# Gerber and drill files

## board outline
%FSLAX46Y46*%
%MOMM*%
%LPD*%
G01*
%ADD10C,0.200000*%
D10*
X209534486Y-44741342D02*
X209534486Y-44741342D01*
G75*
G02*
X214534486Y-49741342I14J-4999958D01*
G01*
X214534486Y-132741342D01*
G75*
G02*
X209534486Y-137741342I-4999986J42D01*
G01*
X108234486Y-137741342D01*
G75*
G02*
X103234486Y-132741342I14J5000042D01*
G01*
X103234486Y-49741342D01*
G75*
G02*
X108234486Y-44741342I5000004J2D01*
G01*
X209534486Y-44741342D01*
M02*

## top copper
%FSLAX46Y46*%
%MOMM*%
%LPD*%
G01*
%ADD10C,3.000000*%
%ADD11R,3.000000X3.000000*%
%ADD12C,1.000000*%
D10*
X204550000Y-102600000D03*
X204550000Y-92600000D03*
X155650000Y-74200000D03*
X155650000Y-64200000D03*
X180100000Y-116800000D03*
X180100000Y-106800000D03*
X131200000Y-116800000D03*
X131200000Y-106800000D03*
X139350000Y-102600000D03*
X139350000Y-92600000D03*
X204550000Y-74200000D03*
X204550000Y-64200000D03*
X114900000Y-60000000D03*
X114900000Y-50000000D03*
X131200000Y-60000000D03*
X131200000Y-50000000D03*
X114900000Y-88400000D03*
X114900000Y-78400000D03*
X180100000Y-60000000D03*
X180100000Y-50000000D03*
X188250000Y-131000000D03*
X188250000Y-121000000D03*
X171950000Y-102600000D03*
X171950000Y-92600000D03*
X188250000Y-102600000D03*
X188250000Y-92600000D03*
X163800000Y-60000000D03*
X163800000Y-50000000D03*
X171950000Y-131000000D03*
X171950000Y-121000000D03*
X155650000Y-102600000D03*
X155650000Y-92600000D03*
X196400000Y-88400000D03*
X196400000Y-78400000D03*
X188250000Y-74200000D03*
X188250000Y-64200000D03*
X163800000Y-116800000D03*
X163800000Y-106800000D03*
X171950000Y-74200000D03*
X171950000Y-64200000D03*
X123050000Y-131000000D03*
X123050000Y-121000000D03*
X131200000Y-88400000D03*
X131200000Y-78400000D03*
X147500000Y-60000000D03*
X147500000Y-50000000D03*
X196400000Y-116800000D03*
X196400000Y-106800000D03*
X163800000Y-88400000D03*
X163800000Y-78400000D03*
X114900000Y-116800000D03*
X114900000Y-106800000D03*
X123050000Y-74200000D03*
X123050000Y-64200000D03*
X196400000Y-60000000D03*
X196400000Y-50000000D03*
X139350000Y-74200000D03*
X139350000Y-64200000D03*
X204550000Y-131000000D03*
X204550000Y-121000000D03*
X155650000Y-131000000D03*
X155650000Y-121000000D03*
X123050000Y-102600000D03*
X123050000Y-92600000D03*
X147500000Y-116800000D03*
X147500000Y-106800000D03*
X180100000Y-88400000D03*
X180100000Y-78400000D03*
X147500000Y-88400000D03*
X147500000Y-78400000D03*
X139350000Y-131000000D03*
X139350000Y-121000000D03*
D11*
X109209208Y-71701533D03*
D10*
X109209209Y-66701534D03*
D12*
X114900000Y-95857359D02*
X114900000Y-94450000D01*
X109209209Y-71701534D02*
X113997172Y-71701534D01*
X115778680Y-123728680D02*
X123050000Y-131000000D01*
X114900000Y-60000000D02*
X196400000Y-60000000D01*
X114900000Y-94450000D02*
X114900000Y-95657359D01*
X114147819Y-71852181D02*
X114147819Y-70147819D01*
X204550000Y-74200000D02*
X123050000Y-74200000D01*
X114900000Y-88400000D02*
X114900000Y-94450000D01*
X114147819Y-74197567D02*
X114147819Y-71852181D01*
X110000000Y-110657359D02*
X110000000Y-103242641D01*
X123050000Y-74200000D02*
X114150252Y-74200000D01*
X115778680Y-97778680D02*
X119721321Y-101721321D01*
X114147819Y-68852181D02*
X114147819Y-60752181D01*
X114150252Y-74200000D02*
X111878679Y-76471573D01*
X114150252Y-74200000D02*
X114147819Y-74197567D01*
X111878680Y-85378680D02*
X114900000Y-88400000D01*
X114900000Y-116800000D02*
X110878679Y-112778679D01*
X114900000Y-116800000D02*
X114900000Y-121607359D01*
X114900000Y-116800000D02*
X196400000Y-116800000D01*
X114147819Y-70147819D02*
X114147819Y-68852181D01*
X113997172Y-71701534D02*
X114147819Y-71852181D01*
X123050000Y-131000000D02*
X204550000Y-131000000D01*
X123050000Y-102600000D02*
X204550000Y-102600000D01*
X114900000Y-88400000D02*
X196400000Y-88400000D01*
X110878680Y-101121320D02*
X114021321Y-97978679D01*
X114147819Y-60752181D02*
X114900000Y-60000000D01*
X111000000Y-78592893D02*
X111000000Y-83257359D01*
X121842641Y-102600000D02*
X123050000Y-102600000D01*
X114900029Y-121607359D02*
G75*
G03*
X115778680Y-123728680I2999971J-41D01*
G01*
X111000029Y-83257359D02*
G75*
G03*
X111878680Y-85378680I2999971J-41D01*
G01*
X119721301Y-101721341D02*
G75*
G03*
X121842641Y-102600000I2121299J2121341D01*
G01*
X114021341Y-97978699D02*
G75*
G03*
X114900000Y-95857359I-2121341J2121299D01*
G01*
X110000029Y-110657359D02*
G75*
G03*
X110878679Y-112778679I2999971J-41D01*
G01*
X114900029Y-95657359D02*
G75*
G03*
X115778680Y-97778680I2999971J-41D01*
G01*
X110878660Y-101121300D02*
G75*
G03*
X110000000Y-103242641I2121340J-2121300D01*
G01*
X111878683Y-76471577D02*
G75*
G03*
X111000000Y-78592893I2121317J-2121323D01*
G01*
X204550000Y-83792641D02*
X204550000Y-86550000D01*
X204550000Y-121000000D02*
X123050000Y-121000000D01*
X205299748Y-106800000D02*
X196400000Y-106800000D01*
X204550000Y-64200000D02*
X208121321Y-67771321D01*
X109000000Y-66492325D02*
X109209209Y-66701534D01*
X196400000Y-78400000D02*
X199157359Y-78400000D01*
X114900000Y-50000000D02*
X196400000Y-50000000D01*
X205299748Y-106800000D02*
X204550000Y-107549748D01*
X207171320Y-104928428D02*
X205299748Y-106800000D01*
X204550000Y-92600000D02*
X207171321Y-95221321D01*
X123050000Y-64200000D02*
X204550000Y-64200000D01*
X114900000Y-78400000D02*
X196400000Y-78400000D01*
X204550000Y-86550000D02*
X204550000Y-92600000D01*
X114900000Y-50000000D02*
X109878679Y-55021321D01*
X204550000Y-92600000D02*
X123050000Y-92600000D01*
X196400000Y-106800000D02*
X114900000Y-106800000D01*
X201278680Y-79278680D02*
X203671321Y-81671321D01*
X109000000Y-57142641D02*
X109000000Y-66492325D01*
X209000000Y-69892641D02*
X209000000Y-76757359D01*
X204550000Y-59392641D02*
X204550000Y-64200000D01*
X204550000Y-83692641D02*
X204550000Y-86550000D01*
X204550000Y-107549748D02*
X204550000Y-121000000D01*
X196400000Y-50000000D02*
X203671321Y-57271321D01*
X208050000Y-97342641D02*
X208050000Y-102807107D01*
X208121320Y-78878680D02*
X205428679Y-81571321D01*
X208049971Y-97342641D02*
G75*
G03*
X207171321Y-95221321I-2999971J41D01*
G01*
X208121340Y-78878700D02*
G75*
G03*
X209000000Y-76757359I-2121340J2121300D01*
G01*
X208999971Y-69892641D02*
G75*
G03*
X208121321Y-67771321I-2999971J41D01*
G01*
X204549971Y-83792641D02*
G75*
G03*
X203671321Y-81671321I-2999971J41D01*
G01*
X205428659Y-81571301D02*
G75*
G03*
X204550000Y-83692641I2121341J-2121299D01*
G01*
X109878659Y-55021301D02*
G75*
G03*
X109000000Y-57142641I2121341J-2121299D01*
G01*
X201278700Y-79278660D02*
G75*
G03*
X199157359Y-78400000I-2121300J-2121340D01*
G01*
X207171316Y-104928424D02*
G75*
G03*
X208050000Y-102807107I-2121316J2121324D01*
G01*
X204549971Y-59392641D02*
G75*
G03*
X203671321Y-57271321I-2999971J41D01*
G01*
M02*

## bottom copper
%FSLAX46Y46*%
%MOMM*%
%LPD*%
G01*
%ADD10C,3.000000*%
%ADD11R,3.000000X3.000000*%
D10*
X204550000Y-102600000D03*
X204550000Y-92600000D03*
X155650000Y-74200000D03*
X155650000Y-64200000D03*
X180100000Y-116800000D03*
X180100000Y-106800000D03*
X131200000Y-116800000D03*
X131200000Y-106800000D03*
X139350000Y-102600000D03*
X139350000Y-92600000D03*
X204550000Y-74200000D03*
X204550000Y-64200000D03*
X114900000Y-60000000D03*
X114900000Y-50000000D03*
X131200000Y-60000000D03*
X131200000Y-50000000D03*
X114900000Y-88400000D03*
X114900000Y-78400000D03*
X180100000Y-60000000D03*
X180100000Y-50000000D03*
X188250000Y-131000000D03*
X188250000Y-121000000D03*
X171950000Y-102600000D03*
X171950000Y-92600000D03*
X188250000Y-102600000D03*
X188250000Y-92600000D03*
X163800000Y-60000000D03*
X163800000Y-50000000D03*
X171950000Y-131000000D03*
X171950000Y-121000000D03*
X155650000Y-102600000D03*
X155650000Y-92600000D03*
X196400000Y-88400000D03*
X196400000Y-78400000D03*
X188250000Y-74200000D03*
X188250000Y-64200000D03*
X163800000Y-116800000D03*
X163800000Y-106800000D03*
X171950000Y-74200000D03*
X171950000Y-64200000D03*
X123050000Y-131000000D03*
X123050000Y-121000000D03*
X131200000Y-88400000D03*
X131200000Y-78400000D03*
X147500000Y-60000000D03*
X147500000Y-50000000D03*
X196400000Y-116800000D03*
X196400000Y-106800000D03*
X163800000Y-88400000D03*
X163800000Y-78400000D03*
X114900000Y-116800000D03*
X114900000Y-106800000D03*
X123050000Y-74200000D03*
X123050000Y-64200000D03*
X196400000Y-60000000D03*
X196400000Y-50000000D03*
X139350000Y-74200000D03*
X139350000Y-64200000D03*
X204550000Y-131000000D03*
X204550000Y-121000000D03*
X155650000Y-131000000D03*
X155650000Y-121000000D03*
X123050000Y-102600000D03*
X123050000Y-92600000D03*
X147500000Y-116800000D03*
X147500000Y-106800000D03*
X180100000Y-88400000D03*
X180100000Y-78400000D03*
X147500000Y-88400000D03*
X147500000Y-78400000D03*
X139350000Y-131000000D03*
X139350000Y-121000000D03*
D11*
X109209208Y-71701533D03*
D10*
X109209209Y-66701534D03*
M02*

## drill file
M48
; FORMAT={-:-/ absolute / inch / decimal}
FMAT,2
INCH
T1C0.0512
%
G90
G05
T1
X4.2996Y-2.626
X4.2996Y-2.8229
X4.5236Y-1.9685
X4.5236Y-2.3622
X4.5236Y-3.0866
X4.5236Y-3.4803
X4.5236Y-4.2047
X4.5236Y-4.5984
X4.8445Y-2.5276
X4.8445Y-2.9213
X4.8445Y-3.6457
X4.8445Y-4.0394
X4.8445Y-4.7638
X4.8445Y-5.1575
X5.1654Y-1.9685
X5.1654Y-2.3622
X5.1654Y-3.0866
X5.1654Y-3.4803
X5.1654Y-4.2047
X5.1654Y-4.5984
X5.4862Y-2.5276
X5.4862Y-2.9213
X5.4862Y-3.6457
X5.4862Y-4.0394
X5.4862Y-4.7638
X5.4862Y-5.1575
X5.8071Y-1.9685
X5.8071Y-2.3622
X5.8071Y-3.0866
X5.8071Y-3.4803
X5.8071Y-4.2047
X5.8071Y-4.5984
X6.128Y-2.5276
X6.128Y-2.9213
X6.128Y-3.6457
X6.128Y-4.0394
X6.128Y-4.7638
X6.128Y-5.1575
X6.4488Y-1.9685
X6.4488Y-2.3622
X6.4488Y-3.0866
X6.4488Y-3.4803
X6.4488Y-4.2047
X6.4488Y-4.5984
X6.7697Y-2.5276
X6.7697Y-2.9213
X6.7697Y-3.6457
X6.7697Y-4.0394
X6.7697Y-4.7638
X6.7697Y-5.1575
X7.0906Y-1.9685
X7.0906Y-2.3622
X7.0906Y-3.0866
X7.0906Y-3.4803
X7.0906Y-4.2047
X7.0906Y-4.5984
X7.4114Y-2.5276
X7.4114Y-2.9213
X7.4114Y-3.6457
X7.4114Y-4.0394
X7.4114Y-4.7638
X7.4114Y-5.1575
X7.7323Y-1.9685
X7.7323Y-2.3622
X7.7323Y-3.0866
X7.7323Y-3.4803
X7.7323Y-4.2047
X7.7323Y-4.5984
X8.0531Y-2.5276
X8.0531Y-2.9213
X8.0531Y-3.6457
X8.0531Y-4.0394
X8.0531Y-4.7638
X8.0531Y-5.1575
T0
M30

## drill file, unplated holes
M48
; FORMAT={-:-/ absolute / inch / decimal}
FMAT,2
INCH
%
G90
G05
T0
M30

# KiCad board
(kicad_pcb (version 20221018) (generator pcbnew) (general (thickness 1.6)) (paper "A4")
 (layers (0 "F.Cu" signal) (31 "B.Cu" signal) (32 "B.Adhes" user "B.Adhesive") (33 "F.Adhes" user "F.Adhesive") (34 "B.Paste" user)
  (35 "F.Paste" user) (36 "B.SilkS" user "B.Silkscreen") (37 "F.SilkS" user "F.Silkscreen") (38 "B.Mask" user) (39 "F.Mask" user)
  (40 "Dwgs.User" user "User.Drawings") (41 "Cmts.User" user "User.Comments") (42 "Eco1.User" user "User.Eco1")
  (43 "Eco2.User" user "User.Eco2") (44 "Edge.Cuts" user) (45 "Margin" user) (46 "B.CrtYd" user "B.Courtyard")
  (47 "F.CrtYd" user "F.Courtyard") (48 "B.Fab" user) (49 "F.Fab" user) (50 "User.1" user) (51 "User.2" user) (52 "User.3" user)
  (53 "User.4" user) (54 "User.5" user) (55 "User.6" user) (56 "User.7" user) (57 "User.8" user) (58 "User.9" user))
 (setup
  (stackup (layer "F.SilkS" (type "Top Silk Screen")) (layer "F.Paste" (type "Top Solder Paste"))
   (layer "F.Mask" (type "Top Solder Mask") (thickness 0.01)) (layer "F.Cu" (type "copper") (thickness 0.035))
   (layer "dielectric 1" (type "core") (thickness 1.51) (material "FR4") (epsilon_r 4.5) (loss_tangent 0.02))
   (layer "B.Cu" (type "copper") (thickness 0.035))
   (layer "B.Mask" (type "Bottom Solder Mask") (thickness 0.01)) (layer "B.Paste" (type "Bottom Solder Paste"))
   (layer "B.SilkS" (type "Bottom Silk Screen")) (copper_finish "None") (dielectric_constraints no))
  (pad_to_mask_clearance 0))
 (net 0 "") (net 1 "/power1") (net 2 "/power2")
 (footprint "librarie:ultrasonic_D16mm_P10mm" (layer "F.Cu") (at 204.55 97.6)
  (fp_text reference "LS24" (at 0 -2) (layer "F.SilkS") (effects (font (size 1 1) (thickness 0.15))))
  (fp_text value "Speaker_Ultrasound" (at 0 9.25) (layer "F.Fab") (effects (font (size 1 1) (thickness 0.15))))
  (pad "1" thru_hole circle (at 0 5) (size 3 3) (drill 1.3) (layers "*.Cu" "*.Mask") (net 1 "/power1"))
  (pad "2" thru_hole circle (at 0 -5) (size 3 3) (drill 1.3) (layers "*.Cu" "*.Mask") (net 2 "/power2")))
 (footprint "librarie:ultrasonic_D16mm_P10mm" (layer "F.Cu") (at 155.65 69.2)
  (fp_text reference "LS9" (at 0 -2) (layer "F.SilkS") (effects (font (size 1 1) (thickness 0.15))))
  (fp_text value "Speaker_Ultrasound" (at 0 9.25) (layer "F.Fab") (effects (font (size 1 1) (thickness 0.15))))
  (pad "1" thru_hole circle (at 0 5) (size 3 3) (drill 1.3) (layers "*.Cu" "*.Mask") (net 1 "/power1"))
  (pad "2" thru_hole circle (at 0 -5) (size 3 3) (drill 1.3) (layers "*.Cu" "*.Mask") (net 2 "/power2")))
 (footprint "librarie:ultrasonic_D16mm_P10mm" (layer "F.Cu") (at 180.1 111.8)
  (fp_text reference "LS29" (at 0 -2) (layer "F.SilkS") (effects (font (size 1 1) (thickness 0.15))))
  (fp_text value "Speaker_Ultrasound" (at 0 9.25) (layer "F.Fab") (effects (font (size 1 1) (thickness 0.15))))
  (pad "1" thru_hole circle (at 0 5) (size 3 3) (drill 1.3) (layers "*.Cu" "*.Mask") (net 1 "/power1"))
  (pad "2" thru_hole circle (at 0 -5) (size 3 3) (drill 1.3) (layers "*.Cu" "*.Mask") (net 2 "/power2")))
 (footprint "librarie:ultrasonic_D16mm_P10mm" (layer "F.Cu") (at 131.2 111.8)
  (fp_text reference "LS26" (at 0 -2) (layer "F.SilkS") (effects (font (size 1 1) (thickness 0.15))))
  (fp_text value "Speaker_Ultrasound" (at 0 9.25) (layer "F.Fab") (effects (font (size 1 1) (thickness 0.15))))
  (pad "1" thru_hole circle (at 0 5) (size 3 3) (drill 1.3) (layers "*.Cu" "*.Mask") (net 1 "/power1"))
  (pad "2" thru_hole circle (at 0 -5) (size 3 3) (drill 1.3) (layers "*.Cu" "*.Mask") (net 2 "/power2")))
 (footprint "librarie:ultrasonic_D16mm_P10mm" (layer "F.Cu") (at 139.35 97.6)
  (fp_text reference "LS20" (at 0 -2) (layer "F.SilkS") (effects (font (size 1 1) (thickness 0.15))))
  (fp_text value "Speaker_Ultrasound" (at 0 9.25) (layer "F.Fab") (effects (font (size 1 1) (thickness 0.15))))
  (pad "1" thru_hole circle (at 0 5) (size 3 3) (drill 1.3) (layers "*.Cu" "*.Mask") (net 1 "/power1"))
  (pad "2" thru_hole circle (at 0 -5) (size 3 3) (drill 1.3) (layers "*.Cu" "*.Mask") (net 2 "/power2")))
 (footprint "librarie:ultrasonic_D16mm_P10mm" (layer "F.Cu") (at 204.55 69.2)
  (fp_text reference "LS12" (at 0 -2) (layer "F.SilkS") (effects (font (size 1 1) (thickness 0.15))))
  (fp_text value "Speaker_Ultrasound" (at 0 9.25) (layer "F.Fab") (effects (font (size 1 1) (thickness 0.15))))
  (pad "1" thru_hole circle (at 0 5) (size 3 3) (drill 1.3) (layers "*.Cu" "*.Mask") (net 1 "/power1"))
  (pad "2" thru_hole circle (at 0 -5) (size 3 3) (drill 1.3) (layers "*.Cu" "*.Mask") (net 2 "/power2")))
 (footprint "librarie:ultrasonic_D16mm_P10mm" (layer "F.Cu") (at 114.9 55)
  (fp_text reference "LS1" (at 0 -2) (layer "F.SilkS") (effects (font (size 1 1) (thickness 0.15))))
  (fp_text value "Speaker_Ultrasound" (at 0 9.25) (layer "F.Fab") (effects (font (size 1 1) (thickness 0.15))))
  (pad "1" thru_hole circle (at 0 5) (size 3 3) (drill 1.3) (layers "*.Cu" "*.Mask") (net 1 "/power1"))
  (pad "2" thru_hole circle (at 0 -5) (size 3 3) (drill 1.3) (layers "*.Cu" "*.Mask") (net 2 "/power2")))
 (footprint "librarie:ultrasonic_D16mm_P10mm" (layer "F.Cu") (at 131.2 55)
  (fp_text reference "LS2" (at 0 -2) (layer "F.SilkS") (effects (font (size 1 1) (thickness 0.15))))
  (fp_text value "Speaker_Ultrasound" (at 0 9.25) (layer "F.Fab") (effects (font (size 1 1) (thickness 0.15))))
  (pad "1" thru_hole circle (at 0 5) (size 3 3) (drill 1.3) (layers "*.Cu" "*.Mask") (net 1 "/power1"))
  (pad "2" thru_hole circle (at 0 -5) (size 3 3) (drill 1.3) (layers "*.Cu" "*.Mask") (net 2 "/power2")))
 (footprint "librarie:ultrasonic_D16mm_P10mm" (layer "F.Cu") (at 114.9 83.4)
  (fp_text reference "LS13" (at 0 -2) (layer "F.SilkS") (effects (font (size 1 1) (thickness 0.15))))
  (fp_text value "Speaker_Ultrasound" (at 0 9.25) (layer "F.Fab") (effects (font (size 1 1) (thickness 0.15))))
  (pad "1" thru_hole circle (at 0 5) (size 3 3) (drill 1.3) (layers "*.Cu" "*.Mask") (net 1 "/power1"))
  (pad "2" thru_hole circle (at 0 -5) (size 3 3) (drill 1.3) (layers "*.Cu" "*.Mask") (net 2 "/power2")))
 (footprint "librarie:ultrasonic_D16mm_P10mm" (layer "F.Cu") (at 180.1 55)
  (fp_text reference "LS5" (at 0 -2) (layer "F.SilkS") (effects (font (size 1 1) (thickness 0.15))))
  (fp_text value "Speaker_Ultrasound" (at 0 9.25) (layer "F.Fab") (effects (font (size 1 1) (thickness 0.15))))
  (pad "1" thru_hole circle (at 0 5) (size 3 3) (drill 1.3) (layers "*.Cu" "*.Mask") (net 1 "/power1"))
  (pad "2" thru_hole circle (at 0 -5) (size 3 3) (drill 1.3) (layers "*.Cu" "*.Mask") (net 2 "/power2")))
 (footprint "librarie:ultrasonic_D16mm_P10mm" (layer "F.Cu") (at 188.25 126)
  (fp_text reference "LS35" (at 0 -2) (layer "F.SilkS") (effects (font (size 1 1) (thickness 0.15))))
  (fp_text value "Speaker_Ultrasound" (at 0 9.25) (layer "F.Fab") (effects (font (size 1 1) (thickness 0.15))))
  (pad "1" thru_hole circle (at 0 5) (size 3 3) (drill 1.3) (layers "*.Cu" "*.Mask") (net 1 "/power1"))
  (pad "2" thru_hole circle (at 0 -5) (size 3 3) (drill 1.3) (layers "*.Cu" "*.Mask") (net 2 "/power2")))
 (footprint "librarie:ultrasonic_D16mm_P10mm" (layer "F.Cu") (at 171.95 97.6)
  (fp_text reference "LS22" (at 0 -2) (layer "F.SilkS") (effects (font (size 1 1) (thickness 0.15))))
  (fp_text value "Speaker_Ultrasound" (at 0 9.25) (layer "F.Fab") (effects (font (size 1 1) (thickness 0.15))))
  (pad "1" thru_hole circle (at 0 5) (size 3 3) (drill 1.3) (layers "*.Cu" "*.Mask") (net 1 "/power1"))
  (pad "2" thru_hole circle (at 0 -5) (size 3 3) (drill 1.3) (layers "*.Cu" "*.Mask") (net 2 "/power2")))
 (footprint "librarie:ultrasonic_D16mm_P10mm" (layer "F.Cu") (at 188.25 97.6)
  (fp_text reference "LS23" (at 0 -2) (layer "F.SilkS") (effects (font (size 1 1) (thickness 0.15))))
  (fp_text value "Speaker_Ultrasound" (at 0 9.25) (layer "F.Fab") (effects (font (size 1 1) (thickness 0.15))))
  (pad "1" thru_hole circle (at 0 5) (size 3 3) (drill 1.3) (layers "*.Cu" "*.Mask") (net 1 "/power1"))
  (pad "2" thru_hole circle (at 0 -5) (size 3 3) (drill 1.3) (layers "*.Cu" "*.Mask") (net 2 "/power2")))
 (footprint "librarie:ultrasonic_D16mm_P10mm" (layer "F.Cu") (at 163.8 55)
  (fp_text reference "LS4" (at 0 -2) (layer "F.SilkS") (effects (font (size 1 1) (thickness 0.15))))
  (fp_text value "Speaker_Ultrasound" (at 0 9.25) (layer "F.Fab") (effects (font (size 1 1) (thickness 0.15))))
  (pad "1" thru_hole circle (at 0 5) (size 3 3) (drill 1.3) (layers "*.Cu" "*.Mask") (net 1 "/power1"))
  (pad "2" thru_hole circle (at 0 -5) (size 3 3) (drill 1.3) (layers "*.Cu" "*.Mask") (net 2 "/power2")))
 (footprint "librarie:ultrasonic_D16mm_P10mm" (layer "F.Cu") (at 171.95 126)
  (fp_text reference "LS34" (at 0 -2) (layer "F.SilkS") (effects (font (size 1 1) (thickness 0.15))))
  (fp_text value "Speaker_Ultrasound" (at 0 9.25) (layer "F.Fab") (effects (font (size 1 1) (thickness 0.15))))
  (pad "1" thru_hole circle (at 0 5) (size 3 3) (drill 1.3) (layers "*.Cu" "*.Mask") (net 1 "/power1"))
  (pad "2" thru_hole circle (at 0 -5) (size 3 3) (drill 1.3) (layers "*.Cu" "*.Mask") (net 2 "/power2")))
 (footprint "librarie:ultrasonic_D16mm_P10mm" (layer "F.Cu") (at 155.65 97.6)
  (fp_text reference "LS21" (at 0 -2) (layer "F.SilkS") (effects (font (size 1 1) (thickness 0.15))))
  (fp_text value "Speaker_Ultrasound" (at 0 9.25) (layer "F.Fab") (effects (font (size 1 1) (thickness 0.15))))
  (pad "1" thru_hole circle (at 0 5) (size 3 3) (drill 1.3) (layers "*.Cu" "*.Mask") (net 1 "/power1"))
  (pad "2" thru_hole circle (at 0 -5) (size 3 3) (drill 1.3) (layers "*.Cu" "*.Mask") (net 2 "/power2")))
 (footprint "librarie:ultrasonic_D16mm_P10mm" (layer "F.Cu") (at 196.4 83.4)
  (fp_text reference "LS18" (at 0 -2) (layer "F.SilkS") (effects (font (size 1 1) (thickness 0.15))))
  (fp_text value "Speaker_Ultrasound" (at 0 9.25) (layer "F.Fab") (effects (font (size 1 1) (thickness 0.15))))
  (pad "1" thru_hole circle (at 0 5) (size 3 3) (drill 1.3) (layers "*.Cu" "*.Mask") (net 1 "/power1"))
  (pad "2" thru_hole circle (at 0 -5) (size 3 3) (drill 1.3) (layers "*.Cu" "*.Mask") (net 2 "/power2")))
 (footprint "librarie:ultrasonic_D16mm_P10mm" (layer "F.Cu") (at 188.25 69.2)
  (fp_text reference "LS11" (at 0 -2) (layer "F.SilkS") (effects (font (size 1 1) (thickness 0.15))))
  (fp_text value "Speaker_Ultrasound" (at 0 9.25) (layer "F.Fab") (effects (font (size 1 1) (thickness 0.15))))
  (pad "1" thru_hole circle (at 0 5) (size 3 3) (drill 1.3) (layers "*.Cu" "*.Mask") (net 1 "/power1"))
  (pad "2" thru_hole circle (at 0 -5) (size 3 3) (drill 1.3) (layers "*.Cu" "*.Mask") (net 2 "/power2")))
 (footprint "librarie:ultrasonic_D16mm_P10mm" (layer "F.Cu") (at 163.8 111.8)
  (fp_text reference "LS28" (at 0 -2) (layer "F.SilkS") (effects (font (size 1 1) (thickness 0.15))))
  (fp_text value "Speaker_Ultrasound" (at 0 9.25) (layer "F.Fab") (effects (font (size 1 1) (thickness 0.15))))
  (pad "1" thru_hole circle (at 0 5) (size 3 3) (drill 1.3) (layers "*.Cu" "*.Mask") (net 1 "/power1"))
  (pad "2" thru_hole circle (at 0 -5) (size 3 3) (drill 1.3) (layers "*.Cu" "*.Mask") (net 2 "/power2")))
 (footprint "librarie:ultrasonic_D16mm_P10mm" (layer "F.Cu") (at 171.95 69.2)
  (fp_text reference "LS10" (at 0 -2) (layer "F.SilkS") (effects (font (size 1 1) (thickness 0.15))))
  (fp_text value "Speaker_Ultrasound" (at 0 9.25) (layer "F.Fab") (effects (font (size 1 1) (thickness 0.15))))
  (pad "1" thru_hole circle (at 0 5) (size 3 3) (drill 1.3) (layers "*.Cu" "*.Mask") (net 1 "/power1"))
  (pad "2" thru_hole circle (at 0 -5) (size 3 3) (drill 1.3) (layers "*.Cu" "*.Mask") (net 2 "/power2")))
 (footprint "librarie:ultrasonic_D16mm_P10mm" (layer "F.Cu") (at 123.05 126)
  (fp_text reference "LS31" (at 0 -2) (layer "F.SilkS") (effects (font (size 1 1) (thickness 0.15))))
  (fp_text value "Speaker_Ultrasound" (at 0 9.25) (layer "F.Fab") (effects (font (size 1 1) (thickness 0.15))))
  (pad "1" thru_hole circle (at 0 5) (size 3 3) (drill 1.3) (layers "*.Cu" "*.Mask") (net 1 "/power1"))
  (pad "2" thru_hole circle (at 0 -5) (size 3 3) (drill 1.3) (layers "*.Cu" "*.Mask") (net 2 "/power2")))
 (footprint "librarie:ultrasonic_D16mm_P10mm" (layer "F.Cu") (at 131.2 83.4)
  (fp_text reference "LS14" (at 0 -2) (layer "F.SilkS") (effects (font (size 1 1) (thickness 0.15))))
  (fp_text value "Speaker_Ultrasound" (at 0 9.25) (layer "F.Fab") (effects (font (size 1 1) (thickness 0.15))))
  (pad "1" thru_hole circle (at 0 5) (size 3 3) (drill 1.3) (layers "*.Cu" "*.Mask") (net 1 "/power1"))
  (pad "2" thru_hole circle (at 0 -5) (size 3 3) (drill 1.3) (layers "*.Cu" "*.Mask") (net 2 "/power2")))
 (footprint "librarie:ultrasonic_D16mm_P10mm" (layer "F.Cu") (at 147.5 55)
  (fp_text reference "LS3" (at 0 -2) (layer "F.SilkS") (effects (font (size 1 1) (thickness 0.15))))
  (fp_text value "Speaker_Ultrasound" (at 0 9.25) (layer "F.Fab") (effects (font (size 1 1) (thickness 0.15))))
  (pad "1" thru_hole circle (at 0 5) (size 3 3) (drill 1.3) (layers "*.Cu" "*.Mask") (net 1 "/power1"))
  (pad "2" thru_hole circle (at 0 -5) (size 3 3) (drill 1.3) (layers "*.Cu" "*.Mask") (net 2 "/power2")))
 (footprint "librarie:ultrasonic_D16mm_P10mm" (layer "F.Cu") (at 196.4 111.8)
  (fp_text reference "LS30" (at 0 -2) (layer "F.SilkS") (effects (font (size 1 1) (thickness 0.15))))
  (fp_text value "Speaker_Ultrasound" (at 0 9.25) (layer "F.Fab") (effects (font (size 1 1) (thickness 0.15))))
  (pad "1" thru_hole circle (at 0 5) (size 3 3) (drill 1.3) (layers "*.Cu" "*.Mask") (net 1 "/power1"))
  (pad "2" thru_hole circle (at 0 -5) (size 3 3) (drill 1.3) (layers "*.Cu" "*.Mask") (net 2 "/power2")))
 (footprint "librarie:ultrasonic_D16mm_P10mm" (layer "F.Cu") (at 163.8 83.4)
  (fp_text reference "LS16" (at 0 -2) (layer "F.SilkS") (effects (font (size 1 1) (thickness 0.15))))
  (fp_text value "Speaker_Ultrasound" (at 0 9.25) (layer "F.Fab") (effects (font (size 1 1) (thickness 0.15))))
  (pad "1" thru_hole circle (at 0 5) (size 3 3) (drill 1.3) (layers "*.Cu" "*.Mask") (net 1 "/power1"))
  (pad "2" thru_hole circle (at 0 -5) (size 3 3) (drill 1.3) (layers "*.Cu" "*.Mask") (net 2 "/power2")))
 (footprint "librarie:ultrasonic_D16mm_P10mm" (layer "F.Cu") (at 114.9 111.8)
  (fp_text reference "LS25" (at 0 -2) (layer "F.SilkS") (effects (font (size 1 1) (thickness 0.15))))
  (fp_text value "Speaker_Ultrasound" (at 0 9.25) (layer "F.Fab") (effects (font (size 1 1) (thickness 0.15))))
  (pad "1" thru_hole circle (at 0 5) (size 3 3) (drill 1.3) (layers "*.Cu" "*.Mask") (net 1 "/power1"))
  (pad "2" thru_hole circle (at 0 -5) (size 3 3) (drill 1.3) (layers "*.Cu" "*.Mask") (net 2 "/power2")))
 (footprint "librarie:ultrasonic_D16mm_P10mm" (layer "F.Cu") (at 123.05 69.2)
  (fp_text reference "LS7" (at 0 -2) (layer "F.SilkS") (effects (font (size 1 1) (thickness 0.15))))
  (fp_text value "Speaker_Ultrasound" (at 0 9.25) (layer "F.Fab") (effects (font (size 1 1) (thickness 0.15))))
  (pad "1" thru_hole circle (at 0 5) (size 3 3) (drill 1.3) (layers "*.Cu" "*.Mask") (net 1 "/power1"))
  (pad "2" thru_hole circle (at 0 -5) (size 3 3) (drill 1.3) (layers "*.Cu" "*.Mask") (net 2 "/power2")))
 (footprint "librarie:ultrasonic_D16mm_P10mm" (layer "F.Cu") (at 196.4 55)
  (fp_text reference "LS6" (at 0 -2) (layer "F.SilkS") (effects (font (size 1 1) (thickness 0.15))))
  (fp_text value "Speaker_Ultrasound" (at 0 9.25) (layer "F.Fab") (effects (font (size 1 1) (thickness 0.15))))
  (pad "1" thru_hole circle (at 0 5) (size 3 3) (drill 1.3) (layers "*.Cu" "*.Mask") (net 1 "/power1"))
  (pad "2" thru_hole circle (at 0 -5) (size 3 3) (drill 1.3) (layers "*.Cu" "*.Mask") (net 2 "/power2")))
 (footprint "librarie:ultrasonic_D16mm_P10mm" (layer "F.Cu") (at 139.35 69.2)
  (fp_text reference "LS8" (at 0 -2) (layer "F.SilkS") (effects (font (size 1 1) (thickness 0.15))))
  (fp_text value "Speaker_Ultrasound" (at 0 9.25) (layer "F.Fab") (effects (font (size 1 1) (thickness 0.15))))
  (pad "1" thru_hole circle (at 0 5) (size 3 3) (drill 1.3) (layers "*.Cu" "*.Mask") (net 1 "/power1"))
  (pad "2" thru_hole circle (at 0 -5) (size 3 3) (drill 1.3) (layers "*.Cu" "*.Mask") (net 2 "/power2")))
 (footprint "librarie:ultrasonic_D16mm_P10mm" (layer "F.Cu") (at 204.55 126)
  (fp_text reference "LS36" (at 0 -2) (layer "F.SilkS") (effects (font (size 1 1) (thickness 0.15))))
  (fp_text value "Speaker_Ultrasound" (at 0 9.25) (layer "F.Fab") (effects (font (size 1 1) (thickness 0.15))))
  (pad "1" thru_hole circle (at 0 5) (size 3 3) (drill 1.3) (layers "*.Cu" "*.Mask") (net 1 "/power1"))
  (pad "2" thru_hole circle (at 0 -5) (size 3 3) (drill 1.3) (layers "*.Cu" "*.Mask") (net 2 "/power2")))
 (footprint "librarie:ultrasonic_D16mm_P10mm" (layer "F.Cu") (at 155.65 126)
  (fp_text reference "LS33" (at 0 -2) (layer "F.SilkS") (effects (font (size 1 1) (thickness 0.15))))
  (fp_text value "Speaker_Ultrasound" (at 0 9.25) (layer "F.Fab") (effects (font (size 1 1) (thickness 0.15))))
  (pad "1" thru_hole circle (at 0 5) (size 3 3) (drill 1.3) (layers "*.Cu" "*.Mask") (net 1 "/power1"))
  (pad "2" thru_hole circle (at 0 -5) (size 3 3) (drill 1.3) (layers "*.Cu" "*.Mask") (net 2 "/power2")))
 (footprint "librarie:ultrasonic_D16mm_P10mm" (layer "F.Cu") (at 123.05 97.6)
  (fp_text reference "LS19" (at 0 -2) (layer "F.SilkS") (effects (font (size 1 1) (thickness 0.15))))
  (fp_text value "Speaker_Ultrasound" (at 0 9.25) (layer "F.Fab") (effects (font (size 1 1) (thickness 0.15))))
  (pad "1" thru_hole circle (at 0 5) (size 3 3) (drill 1.3) (layers "*.Cu" "*.Mask") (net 1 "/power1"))
  (pad "2" thru_hole circle (at 0 -5) (size 3 3) (drill 1.3) (layers "*.Cu" "*.Mask") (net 2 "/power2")))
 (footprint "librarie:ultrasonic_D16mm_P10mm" (layer "F.Cu") (at 147.5 111.8)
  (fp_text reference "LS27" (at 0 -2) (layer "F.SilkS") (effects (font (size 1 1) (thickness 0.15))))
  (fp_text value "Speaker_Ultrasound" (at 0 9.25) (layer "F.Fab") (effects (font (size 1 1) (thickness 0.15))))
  (pad "1" thru_hole circle (at 0 5) (size 3 3) (drill 1.3) (layers "*.Cu" "*.Mask") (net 1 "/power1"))
  (pad "2" thru_hole circle (at 0 -5) (size 3 3) (drill 1.3) (layers "*.Cu" "*.Mask") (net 2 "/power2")))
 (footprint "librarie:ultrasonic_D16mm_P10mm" (layer "F.Cu") (at 180.1 83.4)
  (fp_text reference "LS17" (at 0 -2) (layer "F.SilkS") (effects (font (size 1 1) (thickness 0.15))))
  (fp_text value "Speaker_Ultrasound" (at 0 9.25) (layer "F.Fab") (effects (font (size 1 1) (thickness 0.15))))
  (pad "1" thru_hole circle (at 0 5) (size 3 3) (drill 1.3) (layers "*.Cu" "*.Mask") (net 1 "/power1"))
  (pad "2" thru_hole circle (at 0 -5) (size 3 3) (drill 1.3) (layers "*.Cu" "*.Mask") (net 2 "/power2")))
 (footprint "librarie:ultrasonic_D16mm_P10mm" (layer "F.Cu") (at 147.5 83.4)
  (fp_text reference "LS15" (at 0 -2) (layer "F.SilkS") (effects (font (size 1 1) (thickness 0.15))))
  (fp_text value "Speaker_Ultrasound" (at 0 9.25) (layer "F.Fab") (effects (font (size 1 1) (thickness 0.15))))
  (pad "1" thru_hole circle (at 0 5) (size 3 3) (drill 1.3) (layers "*.Cu" "*.Mask") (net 1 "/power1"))
  (pad "2" thru_hole circle (at 0 -5) (size 3 3) (drill 1.3) (layers "*.Cu" "*.Mask") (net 2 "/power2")))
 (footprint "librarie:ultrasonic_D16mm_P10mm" (layer "F.Cu") (at 139.35 126)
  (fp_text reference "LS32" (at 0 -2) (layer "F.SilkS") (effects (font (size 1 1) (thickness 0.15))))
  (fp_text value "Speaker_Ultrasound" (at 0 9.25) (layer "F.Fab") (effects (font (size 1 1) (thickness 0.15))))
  (pad "1" thru_hole circle (at 0 5) (size 3 3) (drill 1.3) (layers "*.Cu" "*.Mask") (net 1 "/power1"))
  (pad "2" thru_hole circle (at 0 -5) (size 3 3) (drill 1.3) (layers "*.Cu" "*.Mask") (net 2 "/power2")))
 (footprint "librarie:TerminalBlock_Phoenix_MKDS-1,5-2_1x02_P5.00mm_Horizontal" (layer "F.Cu") (at 109.209209 71.701534 90)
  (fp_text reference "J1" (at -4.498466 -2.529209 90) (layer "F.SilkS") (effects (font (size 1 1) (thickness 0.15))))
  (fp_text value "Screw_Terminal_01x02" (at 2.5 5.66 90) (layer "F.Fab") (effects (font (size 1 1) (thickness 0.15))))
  (pad "1" thru_hole rect (at 0 0 90) (size 3 3) (drill 1.3) (layers "*.Cu" "*.Mask") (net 1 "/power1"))
  (pad "2" thru_hole circle (at 5 0 90) (size 3 3) (drill 1.3) (layers "*.Cu" "*.Mask") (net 2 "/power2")))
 (gr_poly
  (pts
   (arc (start 103.234486 132.741342) (mid 104.698952 136.276876) (end 108.234486 137.741342))
   (arc (start 209.534486 137.741342) (mid 213.07002 136.276876) (end 214.534486 132.741342))
   (arc (start 214.534486 49.741342) (mid 213.07002 46.205808) (end 209.534486 44.741342))
   (arc (start 108.234486 44.741342) (mid 104.698952 46.205808) (end 103.234486 49.741342)))
  (stroke (width 0.2) (type solid)) (fill none) (layer "Edge.Cuts"))
 (segment (start 114.9 95.857359) (end 114.9 94.45) (width 1) (layer "F.Cu") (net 1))
 (segment (start 109.209209 71.701534) (end 113.997172 71.701534) (width 1) (layer "F.Cu") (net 1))
 (segment (start 115.77868 123.72868) (end 123.05 131) (width 1) (layer "F.Cu") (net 1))
 (segment (start 114.9 60) (end 196.4 60) (width 1) (layer "F.Cu") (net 1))
 (segment (start 114.9 94.45) (end 114.9 95.657359) (width 1) (layer "F.Cu") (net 1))
 (segment (start 114.147819 71.852181) (end 114.147819 70.147819) (width 1) (layer "F.Cu") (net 1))
 (segment (start 204.55 74.2) (end 123.05 74.2) (width 1) (layer "F.Cu") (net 1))
 (segment (start 114.9 88.4) (end 114.9 94.45) (width 1) (layer "F.Cu") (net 1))
 (segment (start 114.147819 74.197567) (end 114.147819 71.852181) (width 1) (layer "F.Cu") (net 1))
 (segment (start 110 110.657359) (end 110 103.242641) (width 1) (layer "F.Cu") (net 1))
 (segment (start 123.05 74.2) (end 114.150252 74.2) (width 1) (layer "F.Cu") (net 1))
 (segment (start 115.77868 97.77868) (end 119.721321 101.721321) (width 1) (layer "F.Cu") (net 1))
 (segment (start 114.147819 68.852181) (end 114.147819 60.752181) (width 1) (layer "F.Cu") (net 1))
 (segment (start 114.150252 74.2) (end 111.878679 76.471573) (width 1) (layer "F.Cu") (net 1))
 (segment (start 114.150252 74.2) (end 114.147819 74.197567) (width 1) (layer "F.Cu") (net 1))
 (segment (start 111.87868 85.37868) (end 114.9 88.4) (width 1) (layer "F.Cu") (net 1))
 (segment (start 114.9 116.8) (end 110.878679 112.778679) (width 1) (layer "F.Cu") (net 1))
 (segment (start 114.9 116.8) (end 114.9 121.607359) (width 1) (layer "F.Cu") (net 1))
 (segment (start 114.9 116.8) (end 196.4 116.8) (width 1) (layer "F.Cu") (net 1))
 (segment (start 114.147819 70.147819) (end 114.147819 68.852181) (width 1) (layer "F.Cu") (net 1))
 (segment (start 113.997172 71.701534) (end 114.147819 71.852181) (width 1) (layer "F.Cu") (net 1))
 (segment (start 123.05 131) (end 204.55 131) (width 1) (layer "F.Cu") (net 1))
 (segment (start 123.05 102.6) (end 204.55 102.6) (width 1) (layer "F.Cu") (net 1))
 (segment (start 114.9 88.4) (end 196.4 88.4) (width 1) (layer "F.Cu") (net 1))
 (segment (start 110.87868 101.12132) (end 114.021321 97.978679) (width 1) (layer "F.Cu") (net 1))
 (segment (start 114.147819 60.752181) (end 114.9 60) (width 1) (layer "F.Cu") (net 1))
 (segment (start 111 78.592893) (end 111 83.257359) (width 1) (layer "F.Cu") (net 1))
 (segment (start 121.842641 102.6) (end 123.05 102.6) (width 1) (layer "F.Cu") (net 1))
 (arc (start 115.77868 123.72868) (mid 115.128361 122.75541) (end 114.9 121.607359) (width 1) (layer "F.Cu") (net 1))
 (arc (start 111.87868 85.37868) (mid 111.228361 84.40541) (end 111 83.257359) (width 1) (layer "F.Cu") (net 1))
 (arc (start 119.721321 101.721321) (mid 120.694591 102.371639) (end 121.842641 102.6) (width 1) (layer "F.Cu") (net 1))
 (arc (start 114.9 95.857359) (mid 114.671639 97.005409) (end 114.021321 97.978679) (width 1) (layer "F.Cu") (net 1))
 (arc (start 110 110.657359) (mid 110.228361 111.805409) (end 110.878679 112.778679) (width 1) (layer "F.Cu") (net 1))
 (arc (start 114.9 95.657359) (mid 115.128362 96.80541) (end 115.77868 97.77868) (width 1) (layer "F.Cu") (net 1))
 (arc (start 110 103.242641) (mid 110.228362 102.09459) (end 110.87868 101.12132) (width 1) (layer "F.Cu") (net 1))
 (arc (start 111.878679 76.471573) (mid 111.228361 77.444843) (end 111 78.592893) (width 1) (layer "F.Cu") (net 1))
 (segment (start 204.55 83.792641) (end 204.55 86.55) (width 1) (layer "F.Cu") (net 2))
 (segment (start 204.55 121) (end 123.05 121) (width 1) (layer "F.Cu") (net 2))
 (segment (start 205.299748 106.8) (end 196.4 106.8) (width 1) (layer "F.Cu") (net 2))
 (segment (start 204.55 64.2) (end 208.121321 67.771321) (width 1) (layer "F.Cu") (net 2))
 (segment (start 109 66.492325) (end 109.209209 66.701534) (width 1) (layer "F.Cu") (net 2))
 (segment (start 196.4 78.4) (end 199.157359 78.4) (width 1) (layer "F.Cu") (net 2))
 (segment (start 114.9 50) (end 196.4 50) (width 1) (layer "F.Cu") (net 2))
 (segment (start 205.299748 106.8) (end 204.55 107.549748) (width 1) (layer "F.Cu") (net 2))
 (segment (start 207.17132 104.928428) (end 205.299748 106.8) (width 1) (layer "F.Cu") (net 2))
 (segment (start 204.55 92.6) (end 207.171321 95.221321) (width 1) (layer "F.Cu") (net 2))
 (segment (start 123.05 64.2) (end 204.55 64.2) (width 1) (layer "F.Cu") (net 2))
 (segment (start 114.9 78.4) (end 196.4 78.4) (width 1) (layer "F.Cu") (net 2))
 (segment (start 204.55 86.55) (end 204.55 92.6) (width 1) (layer "F.Cu") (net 2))
 (segment (start 114.9 50) (end 109.878679 55.021321) (width 1) (layer "F.Cu") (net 2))
 (segment (start 204.55 92.6) (end 123.05 92.6) (width 1) (layer "F.Cu") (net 2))
 (segment (start 196.4 106.8) (end 114.9 106.8) (width 1) (layer "F.Cu") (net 2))
 (segment (start 201.27868 79.27868) (end 203.671321 81.671321) (width 1) (layer "F.Cu") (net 2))
 (segment (start 109 57.142641) (end 109 66.492325) (width 1) (layer "F.Cu") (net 2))
 (segment (start 209 69.892641) (end 209 76.757359) (width 1) (layer "F.Cu") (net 2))
 (segment (start 204.55 59.392641) (end 204.55 64.2) (width 1) (layer "F.Cu") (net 2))
 (segment (start 204.55 83.692641) (end 204.55 86.55) (width 1) (layer "F.Cu") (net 2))
 (segment (start 204.55 107.549748) (end 204.55 121) (width 1) (layer "F.Cu") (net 2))
 (segment (start 196.4 50) (end 203.671321 57.271321) (width 1) (layer "F.Cu") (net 2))
 (segment (start 208.05 97.342641) (end 208.05 102.807107) (width 1) (layer "F.Cu") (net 2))
 (segment (start 208.12132 78.87868) (end 205.428679 81.571321) (width 1) (layer "F.Cu") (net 2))
 (arc (start 207.171321 95.221321) (mid 207.821639 96.194591) (end 208.05 97.342641) (width 1) (layer "F.Cu") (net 2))
 (arc (start 209 76.757359) (mid 208.771638 77.90541) (end 208.12132 78.87868) (width 1) (layer "F.Cu") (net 2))
 (arc (start 208.121321 67.771321) (mid 208.771639 68.744591) (end 209 69.892641) (width 1) (layer "F.Cu") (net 2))
 (arc (start 204.55 83.792641) (mid 204.321639 82.644591) (end 203.671321 81.671321) (width 1) (layer "F.Cu") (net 2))
 (arc (start 204.55 83.692641) (mid 204.778361 82.544591) (end 205.428679 81.571321) (width 1) (layer "F.Cu") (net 2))
 (arc (start 109 57.142641) (mid 109.228361 55.994591) (end 109.878679 55.021321) (width 1) (layer "F.Cu") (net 2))
 (arc (start 199.157359 78.4) (mid 200.30541 78.628362) (end 201.27868 79.27868) (width 1) (layer "F.Cu") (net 2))
 (arc (start 207.17132 104.928428) (mid 207.821639 103.955158) (end 208.05 102.807107) (width 1) (layer "F.Cu") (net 2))
 (arc (start 204.55 59.392641) (mid 204.321639 58.244591) (end 203.671321 57.271321) (width 1) (layer "F.Cu") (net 2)))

